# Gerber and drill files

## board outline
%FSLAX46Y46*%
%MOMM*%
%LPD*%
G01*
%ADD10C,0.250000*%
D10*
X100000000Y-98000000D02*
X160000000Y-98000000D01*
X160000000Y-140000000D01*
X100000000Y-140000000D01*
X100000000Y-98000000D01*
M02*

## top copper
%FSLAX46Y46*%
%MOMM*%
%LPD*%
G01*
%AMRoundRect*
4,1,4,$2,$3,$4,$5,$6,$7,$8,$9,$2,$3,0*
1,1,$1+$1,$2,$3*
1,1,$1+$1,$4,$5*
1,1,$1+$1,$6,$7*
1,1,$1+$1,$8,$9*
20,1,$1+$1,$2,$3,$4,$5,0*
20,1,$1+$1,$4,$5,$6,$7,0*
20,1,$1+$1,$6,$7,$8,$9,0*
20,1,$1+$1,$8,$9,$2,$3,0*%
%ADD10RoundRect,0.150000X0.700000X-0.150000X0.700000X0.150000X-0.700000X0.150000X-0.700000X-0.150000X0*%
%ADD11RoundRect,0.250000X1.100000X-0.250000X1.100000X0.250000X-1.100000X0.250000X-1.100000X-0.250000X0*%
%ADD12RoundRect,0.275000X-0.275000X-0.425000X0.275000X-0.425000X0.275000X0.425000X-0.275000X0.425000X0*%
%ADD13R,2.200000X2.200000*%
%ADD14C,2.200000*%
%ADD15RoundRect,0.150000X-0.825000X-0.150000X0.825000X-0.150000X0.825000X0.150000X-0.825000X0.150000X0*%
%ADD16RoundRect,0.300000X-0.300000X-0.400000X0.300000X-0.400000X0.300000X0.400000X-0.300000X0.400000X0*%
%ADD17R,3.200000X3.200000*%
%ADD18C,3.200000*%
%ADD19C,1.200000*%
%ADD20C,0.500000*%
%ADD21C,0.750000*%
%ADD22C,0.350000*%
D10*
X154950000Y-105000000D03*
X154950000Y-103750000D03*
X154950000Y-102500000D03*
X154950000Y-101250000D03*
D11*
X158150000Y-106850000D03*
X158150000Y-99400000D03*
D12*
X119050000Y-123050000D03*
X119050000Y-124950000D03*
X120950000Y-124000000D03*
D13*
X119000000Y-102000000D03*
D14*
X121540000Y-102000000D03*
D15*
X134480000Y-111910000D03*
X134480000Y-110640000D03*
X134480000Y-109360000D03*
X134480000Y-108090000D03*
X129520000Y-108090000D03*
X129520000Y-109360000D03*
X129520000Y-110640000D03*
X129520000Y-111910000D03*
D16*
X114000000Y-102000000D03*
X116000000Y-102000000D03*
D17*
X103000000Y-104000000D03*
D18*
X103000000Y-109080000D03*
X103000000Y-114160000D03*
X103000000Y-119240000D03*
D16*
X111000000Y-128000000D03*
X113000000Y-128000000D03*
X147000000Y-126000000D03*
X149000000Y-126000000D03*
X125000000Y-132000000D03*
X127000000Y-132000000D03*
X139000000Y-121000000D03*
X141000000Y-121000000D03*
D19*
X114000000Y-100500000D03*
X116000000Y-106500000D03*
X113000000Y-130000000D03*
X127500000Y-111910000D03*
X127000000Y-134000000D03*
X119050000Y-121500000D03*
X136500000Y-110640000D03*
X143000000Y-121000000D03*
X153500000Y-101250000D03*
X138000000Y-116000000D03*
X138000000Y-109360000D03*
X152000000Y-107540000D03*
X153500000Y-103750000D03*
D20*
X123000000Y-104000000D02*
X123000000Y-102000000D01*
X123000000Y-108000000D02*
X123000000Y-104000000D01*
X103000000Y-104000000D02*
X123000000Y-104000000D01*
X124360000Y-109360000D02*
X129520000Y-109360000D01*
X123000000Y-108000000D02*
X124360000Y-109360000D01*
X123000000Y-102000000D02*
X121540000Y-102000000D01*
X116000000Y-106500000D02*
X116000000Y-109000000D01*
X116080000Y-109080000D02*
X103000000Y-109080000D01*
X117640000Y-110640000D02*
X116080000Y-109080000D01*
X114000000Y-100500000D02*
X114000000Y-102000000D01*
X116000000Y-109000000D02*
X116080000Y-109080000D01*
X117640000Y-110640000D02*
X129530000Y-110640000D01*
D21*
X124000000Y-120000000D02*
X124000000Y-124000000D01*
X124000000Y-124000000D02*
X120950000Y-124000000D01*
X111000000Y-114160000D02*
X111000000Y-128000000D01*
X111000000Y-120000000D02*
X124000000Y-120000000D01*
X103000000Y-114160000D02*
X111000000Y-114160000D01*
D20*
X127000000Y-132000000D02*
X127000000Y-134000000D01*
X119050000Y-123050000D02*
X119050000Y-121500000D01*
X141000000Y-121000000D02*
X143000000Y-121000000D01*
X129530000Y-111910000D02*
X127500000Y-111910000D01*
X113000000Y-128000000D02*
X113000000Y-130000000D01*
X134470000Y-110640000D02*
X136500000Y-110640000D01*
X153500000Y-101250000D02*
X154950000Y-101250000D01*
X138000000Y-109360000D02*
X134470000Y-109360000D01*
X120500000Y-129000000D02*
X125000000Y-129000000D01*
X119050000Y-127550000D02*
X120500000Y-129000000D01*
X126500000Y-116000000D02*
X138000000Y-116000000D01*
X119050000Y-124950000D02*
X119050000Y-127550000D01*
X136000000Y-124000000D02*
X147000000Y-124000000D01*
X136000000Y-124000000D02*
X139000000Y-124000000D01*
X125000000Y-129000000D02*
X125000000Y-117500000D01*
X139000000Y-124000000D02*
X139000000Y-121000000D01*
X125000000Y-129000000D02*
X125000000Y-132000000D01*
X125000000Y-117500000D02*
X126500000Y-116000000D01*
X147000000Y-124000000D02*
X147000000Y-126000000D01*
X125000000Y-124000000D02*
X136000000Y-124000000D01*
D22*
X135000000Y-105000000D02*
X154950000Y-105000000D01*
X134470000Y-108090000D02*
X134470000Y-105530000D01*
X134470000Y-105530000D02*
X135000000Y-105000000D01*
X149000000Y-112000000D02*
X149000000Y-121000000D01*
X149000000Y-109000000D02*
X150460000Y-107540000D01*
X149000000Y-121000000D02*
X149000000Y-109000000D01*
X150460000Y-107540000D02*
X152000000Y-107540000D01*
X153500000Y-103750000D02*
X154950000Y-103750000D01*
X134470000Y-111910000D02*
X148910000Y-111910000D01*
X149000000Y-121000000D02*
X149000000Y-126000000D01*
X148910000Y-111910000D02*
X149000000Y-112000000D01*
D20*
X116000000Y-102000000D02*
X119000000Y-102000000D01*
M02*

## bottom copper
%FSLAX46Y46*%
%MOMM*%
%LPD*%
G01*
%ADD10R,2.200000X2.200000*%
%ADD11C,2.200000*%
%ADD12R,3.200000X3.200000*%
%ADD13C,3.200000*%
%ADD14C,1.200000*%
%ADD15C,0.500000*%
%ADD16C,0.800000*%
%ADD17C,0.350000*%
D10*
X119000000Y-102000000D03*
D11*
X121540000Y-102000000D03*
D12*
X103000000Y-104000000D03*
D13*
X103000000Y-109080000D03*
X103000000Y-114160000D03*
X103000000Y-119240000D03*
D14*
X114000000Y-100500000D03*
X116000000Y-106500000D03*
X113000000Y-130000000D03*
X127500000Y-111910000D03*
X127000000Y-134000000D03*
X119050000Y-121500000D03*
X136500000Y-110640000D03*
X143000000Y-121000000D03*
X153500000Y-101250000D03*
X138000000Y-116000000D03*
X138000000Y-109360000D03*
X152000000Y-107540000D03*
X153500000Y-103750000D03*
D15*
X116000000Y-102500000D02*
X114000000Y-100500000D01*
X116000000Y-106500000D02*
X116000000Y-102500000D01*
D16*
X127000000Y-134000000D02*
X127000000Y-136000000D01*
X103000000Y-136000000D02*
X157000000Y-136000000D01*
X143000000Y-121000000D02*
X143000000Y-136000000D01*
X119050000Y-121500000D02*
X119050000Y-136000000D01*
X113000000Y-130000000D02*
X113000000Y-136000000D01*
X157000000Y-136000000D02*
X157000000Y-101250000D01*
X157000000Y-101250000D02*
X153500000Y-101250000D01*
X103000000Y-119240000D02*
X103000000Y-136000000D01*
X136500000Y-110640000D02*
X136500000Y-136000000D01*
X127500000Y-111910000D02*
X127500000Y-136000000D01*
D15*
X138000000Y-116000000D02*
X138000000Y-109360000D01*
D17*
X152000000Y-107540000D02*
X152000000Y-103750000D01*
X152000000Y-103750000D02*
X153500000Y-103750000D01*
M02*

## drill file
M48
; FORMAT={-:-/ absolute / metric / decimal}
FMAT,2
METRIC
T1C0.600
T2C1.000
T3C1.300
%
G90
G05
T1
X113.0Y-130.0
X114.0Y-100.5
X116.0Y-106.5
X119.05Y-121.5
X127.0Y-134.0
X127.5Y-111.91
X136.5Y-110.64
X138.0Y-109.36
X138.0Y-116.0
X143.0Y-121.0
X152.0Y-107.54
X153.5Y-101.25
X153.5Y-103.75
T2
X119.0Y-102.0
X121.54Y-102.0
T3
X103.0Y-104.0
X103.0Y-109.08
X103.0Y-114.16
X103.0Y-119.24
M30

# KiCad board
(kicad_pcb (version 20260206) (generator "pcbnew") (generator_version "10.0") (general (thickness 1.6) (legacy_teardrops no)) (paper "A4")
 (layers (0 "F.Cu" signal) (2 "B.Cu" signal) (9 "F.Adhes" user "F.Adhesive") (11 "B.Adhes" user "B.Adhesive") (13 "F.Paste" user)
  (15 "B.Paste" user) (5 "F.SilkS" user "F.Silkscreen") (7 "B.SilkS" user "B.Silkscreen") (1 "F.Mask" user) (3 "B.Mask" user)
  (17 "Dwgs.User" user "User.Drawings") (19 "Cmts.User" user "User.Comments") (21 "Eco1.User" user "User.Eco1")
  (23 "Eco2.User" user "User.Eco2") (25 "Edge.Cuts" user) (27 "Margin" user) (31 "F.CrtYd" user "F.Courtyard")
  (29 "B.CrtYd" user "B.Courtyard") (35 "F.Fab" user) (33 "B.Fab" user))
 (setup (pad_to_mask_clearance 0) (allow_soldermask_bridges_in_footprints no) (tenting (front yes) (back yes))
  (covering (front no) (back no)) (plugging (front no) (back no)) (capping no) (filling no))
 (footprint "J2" (layer "F.Cu") (at 156.8 103.125 90)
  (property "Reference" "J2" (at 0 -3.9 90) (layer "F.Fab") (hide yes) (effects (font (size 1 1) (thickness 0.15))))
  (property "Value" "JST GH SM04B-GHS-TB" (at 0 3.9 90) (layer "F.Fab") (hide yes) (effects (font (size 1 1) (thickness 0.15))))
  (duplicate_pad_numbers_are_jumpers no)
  (pad "1" smd roundrect (at -1.875 -1.85 90) (size 0.6 1.7) (layers "F.Cu" "F.Mask" "F.Paste") (roundrect_rratio 0.25) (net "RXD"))
  (pad "2" smd roundrect (at -0.625 -1.85 90) (size 0.6 1.7) (layers "F.Cu" "F.Mask" "F.Paste") (roundrect_rratio 0.25) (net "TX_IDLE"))
  (pad "3" smd roundrect (at 0.625 -1.85 90) (size 0.6 1.7) (layers "F.Cu" "F.Mask" "F.Paste") (roundrect_rratio 0.25))
  (pad "4" smd roundrect (at 1.875 -1.85 90) (size 0.6 1.7) (layers "F.Cu" "F.Mask" "F.Paste") (roundrect_rratio 0.25) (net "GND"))
  (pad "MP" smd roundrect (at -3.725 1.35 90) (size 1 2.7) (layers "F.Cu" "F.Mask" "F.Paste") (roundrect_rratio 0.25))
  (pad "MP" smd roundrect (at 3.725 1.35 90) (size 1 2.7) (layers "F.Cu" "F.Mask" "F.Paste") (roundrect_rratio 0.25)))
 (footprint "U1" (layer "F.Cu") (at 120 124)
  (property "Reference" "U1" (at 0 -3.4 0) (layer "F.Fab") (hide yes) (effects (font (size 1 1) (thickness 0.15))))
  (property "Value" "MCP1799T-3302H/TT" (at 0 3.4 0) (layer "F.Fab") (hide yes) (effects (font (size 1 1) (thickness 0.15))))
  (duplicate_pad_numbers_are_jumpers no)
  (pad "1" smd roundrect (at -0.95 -0.95) (size 1.1 1.4) (layers "F.Cu" "F.Mask" "F.Paste") (roundrect_rratio 0.25) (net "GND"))
  (pad "2" smd roundrect (at -0.95 0.95) (size 1.1 1.4) (layers "F.Cu" "F.Mask" "F.Paste") (roundrect_rratio 0.25) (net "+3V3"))
  (pad "3" smd roundrect (at 0.95 0) (size 1.1 1.4) (layers "F.Cu" "F.Mask" "F.Paste") (roundrect_rratio 0.25) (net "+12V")))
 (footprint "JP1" (layer "F.Cu") (at 119 102)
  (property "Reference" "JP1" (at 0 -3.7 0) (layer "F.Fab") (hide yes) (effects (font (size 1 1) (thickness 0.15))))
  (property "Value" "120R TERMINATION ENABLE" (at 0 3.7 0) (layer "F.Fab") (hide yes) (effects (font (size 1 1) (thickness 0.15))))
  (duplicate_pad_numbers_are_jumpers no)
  (pad "1" thru_hole rect (at 0 0) (size 2.2 2.2) (drill 1) (layers "*.Cu" "*.Mask") (remove_unused_layers no) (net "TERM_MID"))
  (pad "2" thru_hole circle (at 2.54 0) (size 2.2 2.2) (drill 1) (layers "*.Cu" "*.Mask") (remove_unused_layers no) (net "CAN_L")))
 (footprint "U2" (layer "F.Cu") (at 132 110 180)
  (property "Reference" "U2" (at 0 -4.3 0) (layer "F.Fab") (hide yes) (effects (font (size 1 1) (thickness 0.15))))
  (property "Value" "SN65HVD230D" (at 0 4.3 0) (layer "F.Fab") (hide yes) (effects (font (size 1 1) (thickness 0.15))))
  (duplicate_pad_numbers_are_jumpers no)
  (pad "1" smd roundrect (at -2.48 -1.91) (size 1.95 0.6) (layers "F.Cu" "F.Mask" "F.Paste") (roundrect_rratio 0.25) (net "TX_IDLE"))
  (pad "2" smd roundrect (at -2.48 -0.64) (size 1.95 0.6) (layers "F.Cu" "F.Mask" "F.Paste") (roundrect_rratio 0.25) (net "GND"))
  (pad "3" smd roundrect (at -2.48 0.64) (size 1.95 0.6) (layers "F.Cu" "F.Mask" "F.Paste") (roundrect_rratio 0.25) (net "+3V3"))
  (pad "4" smd roundrect (at -2.48 1.91) (size 1.95 0.6) (layers "F.Cu" "F.Mask" "F.Paste") (roundrect_rratio 0.25) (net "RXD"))
  (pad "5" smd roundrect (at 2.48 1.91) (size 1.95 0.6) (layers "F.Cu" "F.Mask" "F.Paste") (roundrect_rratio 0.25))
  (pad "6" smd roundrect (at 2.48 0.64) (size 1.95 0.6) (layers "F.Cu" "F.Mask" "F.Paste") (roundrect_rratio 0.25) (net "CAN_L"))
  (pad "7" smd roundrect (at 2.48 -0.64) (size 1.95 0.6) (layers "F.Cu" "F.Mask" "F.Paste") (roundrect_rratio 0.25) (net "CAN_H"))
  (pad "8" smd roundrect (at 2.48 -1.91) (size 1.95 0.6) (layers "F.Cu" "F.Mask" "F.Paste") (roundrect_rratio 0.25) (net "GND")))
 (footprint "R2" (layer "F.Cu") (at 115 102)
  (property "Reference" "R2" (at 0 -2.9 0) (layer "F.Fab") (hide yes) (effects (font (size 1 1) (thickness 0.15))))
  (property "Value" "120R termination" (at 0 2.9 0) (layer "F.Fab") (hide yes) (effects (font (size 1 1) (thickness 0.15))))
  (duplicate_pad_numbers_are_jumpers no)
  (pad "1" smd roundrect (at -1 0) (size 1.2 1.4) (layers "F.Cu" "F.Mask" "F.Paste") (roundrect_rratio 0.25) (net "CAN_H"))
  (pad "2" smd roundrect (at 1 0) (size 1.2 1.4) (layers "F.Cu" "F.Mask" "F.Paste") (roundrect_rratio 0.25) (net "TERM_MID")))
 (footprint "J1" (layer "F.Cu") (at 103 104)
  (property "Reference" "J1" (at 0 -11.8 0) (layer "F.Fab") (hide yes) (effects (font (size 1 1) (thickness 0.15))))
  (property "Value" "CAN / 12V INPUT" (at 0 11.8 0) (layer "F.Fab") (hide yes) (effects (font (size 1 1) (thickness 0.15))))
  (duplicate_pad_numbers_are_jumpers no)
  (pad "1" thru_hole rect (at 0 0) (size 3.2 3.2) (drill 1.3) (layers "*.Cu" "*.Mask") (remove_unused_layers no) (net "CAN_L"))
  (pad "2" thru_hole circle (at 0 5.08) (size 3.2 3.2) (drill 1.3) (layers "*.Cu" "*.Mask") (remove_unused_layers no) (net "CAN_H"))
  (pad "3" thru_hole circle (at 0 10.16) (size 3.2 3.2) (drill 1.3) (layers "*.Cu" "*.Mask") (remove_unused_layers no) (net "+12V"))
  (pad "4" thru_hole circle (at 0 15.24) (size 3.2 3.2) (drill 1.3) (layers "*.Cu" "*.Mask") (remove_unused_layers no) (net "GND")))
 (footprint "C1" (layer "F.Cu") (at 112 128)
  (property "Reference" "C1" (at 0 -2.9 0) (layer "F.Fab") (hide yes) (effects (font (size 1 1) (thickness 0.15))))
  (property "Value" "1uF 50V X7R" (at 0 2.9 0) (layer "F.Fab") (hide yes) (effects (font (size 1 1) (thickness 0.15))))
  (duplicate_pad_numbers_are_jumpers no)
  (pad "1" smd roundrect (at -1 0) (size 1.2 1.4) (layers "F.Cu" "F.Mask" "F.Paste") (roundrect_rratio 0.25) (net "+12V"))
  (pad "2" smd roundrect (at 1 0) (size 1.2 1.4) (layers "F.Cu" "F.Mask" "F.Paste") (roundrect_rratio 0.25) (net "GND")))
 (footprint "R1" (layer "F.Cu") (at 148 126)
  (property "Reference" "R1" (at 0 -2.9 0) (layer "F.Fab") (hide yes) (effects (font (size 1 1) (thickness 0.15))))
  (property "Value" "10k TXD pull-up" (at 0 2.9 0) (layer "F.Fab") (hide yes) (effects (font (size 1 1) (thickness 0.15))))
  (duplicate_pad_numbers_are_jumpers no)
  (pad "1" smd roundrect (at -1 0) (size 1.2 1.4) (layers "F.Cu" "F.Mask" "F.Paste") (roundrect_rratio 0.25) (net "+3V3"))
  (pad "2" smd roundrect (at 1 0) (size 1.2 1.4) (layers "F.Cu" "F.Mask" "F.Paste") (roundrect_rratio 0.25) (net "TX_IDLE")))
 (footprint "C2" (layer "F.Cu") (at 126 132)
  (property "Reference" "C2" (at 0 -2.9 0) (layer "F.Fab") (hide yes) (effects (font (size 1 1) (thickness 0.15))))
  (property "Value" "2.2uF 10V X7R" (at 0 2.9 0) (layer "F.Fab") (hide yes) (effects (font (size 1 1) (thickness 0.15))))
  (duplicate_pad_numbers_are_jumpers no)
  (pad "1" smd roundrect (at -1 0) (size 1.2 1.4) (layers "F.Cu" "F.Mask" "F.Paste") (roundrect_rratio 0.25) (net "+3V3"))
  (pad "2" smd roundrect (at 1 0) (size 1.2 1.4) (layers "F.Cu" "F.Mask" "F.Paste") (roundrect_rratio 0.25) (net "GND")))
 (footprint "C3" (layer "F.Cu") (at 140 121)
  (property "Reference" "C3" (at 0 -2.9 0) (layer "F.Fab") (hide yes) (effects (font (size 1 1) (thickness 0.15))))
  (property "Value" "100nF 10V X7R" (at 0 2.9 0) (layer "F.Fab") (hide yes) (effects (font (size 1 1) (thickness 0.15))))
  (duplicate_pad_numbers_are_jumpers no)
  (pad "1" smd roundrect (at -1 0) (size 1.2 1.4) (layers "F.Cu" "F.Mask" "F.Paste") (roundrect_rratio 0.25) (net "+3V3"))
  (pad "2" smd roundrect (at 1 0) (size 1.2 1.4) (layers "F.Cu" "F.Mask" "F.Paste") (roundrect_rratio 0.25) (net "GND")))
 (gr_rect (start 100 98) (end 160 140) (stroke (width 0.25) (type default)) (fill no) (layer "Edge.Cuts"))
 (segment (start 123 104) (end 123 102) (width 0.5) (layer "F.Cu") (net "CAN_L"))
 (segment (start 123 108) (end 123 104) (width 0.5) (layer "F.Cu") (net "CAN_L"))
 (segment (start 103 104) (end 123 104) (width 0.5) (layer "F.Cu") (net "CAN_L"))
 (segment (start 124.36 109.36) (end 129.52 109.36) (width 0.5) (layer "F.Cu") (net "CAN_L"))
 (segment (start 123 108) (end 124.36 109.36) (width 0.5) (layer "F.Cu") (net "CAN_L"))
 (segment (start 123 102) (end 121.54 102) (width 0.5) (layer "F.Cu") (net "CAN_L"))
 (segment (start 116 106.5) (end 116 109) (width 0.5) (layer "F.Cu") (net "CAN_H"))
 (segment (start 116.08 109.08) (end 103 109.08) (width 0.5) (layer "F.Cu") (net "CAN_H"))
 (segment (start 117.64 110.64) (end 116.08 109.08) (width 0.5) (layer "F.Cu") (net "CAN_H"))
 (segment (start 114 100.5) (end 114 102) (width 0.5) (layer "F.Cu") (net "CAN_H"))
 (segment (start 116 109) (end 116.08 109.08) (width 0.5) (layer "F.Cu") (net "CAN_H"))
 (segment (start 117.64 110.64) (end 129.53 110.64) (width 0.5) (layer "F.Cu") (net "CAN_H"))
 (via (at 114 100.5) (size 1.2) (drill 0.6) (layers "F.Cu" "B.Cu") (capping no) (covering (front no) (back no))
  (plugging (front no) (back no)) (filling no) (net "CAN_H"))
 (via (at 116 106.5) (size 1.2) (drill 0.6) (layers "F.Cu" "B.Cu") (capping no) (covering (front no) (back no))
  (plugging (front no) (back no)) (filling no) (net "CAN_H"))
 (segment (start 116 102.5) (end 114 100.5) (width 0.5) (layer "B.Cu") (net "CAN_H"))
 (segment (start 116 106.5) (end 116 102.5) (width 0.5) (layer "B.Cu") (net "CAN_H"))
 (segment (start 124 120) (end 124 124) (width 0.75) (layer "F.Cu") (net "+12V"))
 (segment (start 124 124) (end 120.95 124) (width 0.75) (layer "F.Cu") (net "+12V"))
 (segment (start 111 114.16) (end 111 128) (width 0.75) (layer "F.Cu") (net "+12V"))
 (segment (start 111 120) (end 124 120) (width 0.75) (layer "F.Cu") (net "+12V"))
 (segment (start 103 114.16) (end 111 114.16) (width 0.75) (layer "F.Cu") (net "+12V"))
 (segment (start 127 132) (end 127 134) (width 0.5) (layer "F.Cu") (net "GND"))
 (segment (start 119.05 123.05) (end 119.05 121.5) (width 0.5) (layer "F.Cu") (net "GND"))
 (segment (start 141 121) (end 143 121) (width 0.5) (layer "F.Cu") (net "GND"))
 (segment (start 129.53 111.91) (end 127.5 111.91) (width 0.5) (layer "F.Cu") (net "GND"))
 (segment (start 113 128) (end 113 130) (width 0.5) (layer "F.Cu") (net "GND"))
 (segment (start 134.47 110.64) (end 136.5 110.64) (width 0.5) (layer "F.Cu") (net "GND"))
 (via (at 113 130) (size 1.2) (drill 0.6) (layers "F.Cu" "B.Cu") (capping no) (covering (front no) (back no))
  (plugging (front no) (back no)) (filling no) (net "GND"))
 (via (at 127.5 111.91) (size 1.2) (drill 0.6) (layers "F.Cu" "B.Cu") (capping no) (covering (front no) (back no))
  (plugging (front no) (back no)) (filling no) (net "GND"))
 (via (at 127 134) (size 1.2) (drill 0.6) (layers "F.Cu" "B.Cu") (capping no) (covering (front no) (back no))
  (plugging (front no) (back no)) (filling no) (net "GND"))
 (via (at 119.05 121.5) (size 1.2) (drill 0.6) (layers "F.Cu" "B.Cu") (capping no) (covering (front no) (back no))
  (plugging (front no) (back no)) (filling no) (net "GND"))
 (via (at 136.5 110.64) (size 1.2) (drill 0.6) (layers "F.Cu" "B.Cu") (capping no) (covering (front no) (back no))
  (plugging (front no) (back no)) (filling no) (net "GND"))
 (via (at 143 121) (size 1.2) (drill 0.6) (layers "F.Cu" "B.Cu") (capping no) (covering (front no) (back no))
  (plugging (front no) (back no)) (filling no) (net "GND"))
 (segment (start 127 134) (end 127 136) (width 0.8) (layer "B.Cu") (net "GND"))
 (segment (start 103 136) (end 157 136) (width 0.8) (layer "B.Cu") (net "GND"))
 (segment (start 143 121) (end 143 136) (width 0.8) (layer "B.Cu") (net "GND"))
 (segment (start 119.05 121.5) (end 119.05 136) (width 0.8) (layer "B.Cu") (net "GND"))
 (segment (start 113 130) (end 113 136) (width 0.8) (layer "B.Cu") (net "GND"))
 (segment (start 157 136) (end 157 101.25) (width 0.8) (layer "B.Cu") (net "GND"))
 (segment (start 157 101.25) (end 153.5 101.25) (width 0.8) (layer "B.Cu") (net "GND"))
 (via (at 153.5 101.25) (size 1.2) (drill 0.6) (layers "F.Cu" "B.Cu") (capping no) (covering (front no) (back no))
  (plugging (front no) (back no)) (filling no) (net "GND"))
 (segment (start 153.5 101.25) (end 154.95 101.25) (width 0.5) (layer "F.Cu") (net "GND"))
 (segment (start 103 119.24) (end 103 136) (width 0.8) (layer "B.Cu") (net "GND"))
 (segment (start 136.5 110.64) (end 136.5 136) (width 0.8) (layer "B.Cu") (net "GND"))
 (segment (start 127.5 111.91) (end 127.5 136) (width 0.8) (layer "B.Cu") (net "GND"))
 (segment (start 138 109.36) (end 134.47 109.36) (width 0.5) (layer "F.Cu") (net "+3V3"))
 (segment (start 120.5 129) (end 125 129) (width 0.5) (layer "F.Cu") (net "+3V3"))
 (segment (start 119.05 127.55) (end 120.5 129) (width 0.5) (layer "F.Cu") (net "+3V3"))
 (segment (start 126.5 116) (end 138 116) (width 0.5) (layer "F.Cu") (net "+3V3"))
 (segment (start 119.05 124.95) (end 119.05 127.55) (width 0.5) (layer "F.Cu") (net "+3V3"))
 (segment (start 136 124) (end 147 124) (width 0.5) (layer "F.Cu") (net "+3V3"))
 (segment (start 136 124) (end 139 124) (width 0.5) (layer "F.Cu") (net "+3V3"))
 (segment (start 125 129) (end 125 117.5) (width 0.5) (layer "F.Cu") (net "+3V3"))
 (segment (start 139 124) (end 139 121) (width 0.5) (layer "F.Cu") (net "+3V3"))
 (segment (start 125 129) (end 125 132) (width 0.5) (layer "F.Cu") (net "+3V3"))
 (segment (start 125 117.5) (end 126.5 116) (width 0.5) (layer "F.Cu") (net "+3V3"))
 (segment (start 147 124) (end 147 126) (width 0.5) (layer "F.Cu") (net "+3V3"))
 (segment (start 125 124) (end 136 124) (width 0.5) (layer "F.Cu") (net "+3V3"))
 (via (at 138 116) (size 1.2) (drill 0.6) (layers "F.Cu" "B.Cu") (capping no) (covering (front no) (back no))
  (plugging (front no) (back no)) (filling no) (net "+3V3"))
 (via (at 138 109.36) (size 1.2) (drill 0.6) (layers "F.Cu" "B.Cu") (capping no) (covering (front no) (back no))
  (plugging (front no) (back no)) (filling no) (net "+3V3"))
 (segment (start 138 116) (end 138 109.36) (width 0.5) (layer "B.Cu") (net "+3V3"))
 (segment (start 135 105) (end 154.95 105) (width 0.35) (layer "F.Cu") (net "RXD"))
 (segment (start 134.47 108.09) (end 134.47 105.53) (width 0.35) (layer "F.Cu") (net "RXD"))
 (segment (start 134.47 105.53) (end 135 105) (width 0.35) (layer "F.Cu") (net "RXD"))
 (segment (start 149 112) (end 149 121) (width 0.35) (layer "F.Cu") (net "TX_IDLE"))
 (segment (start 149 109) (end 150.46 107.54) (width 0.35) (layer "F.Cu") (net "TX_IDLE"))
 (segment (start 149 121) (end 149 109) (width 0.35) (layer "F.Cu") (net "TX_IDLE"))
 (segment (start 150.46 107.54) (end 152 107.54) (width 0.35) (layer "F.Cu") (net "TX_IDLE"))
 (via (at 152 107.54) (size 1.2) (drill 0.6) (layers "F.Cu" "B.Cu") (capping no) (covering (front no) (back no))
  (plugging (front no) (back no)) (filling no) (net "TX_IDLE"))
 (segment (start 152 107.54) (end 152 103.75) (width 0.35) (layer "B.Cu") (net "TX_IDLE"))
 (segment (start 152 103.75) (end 153.5 103.75) (width 0.35) (layer "B.Cu") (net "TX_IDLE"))
 (via (at 153.5 103.75) (size 1.2) (drill 0.6) (layers "F.Cu" "B.Cu") (capping no) (covering (front no) (back no))
  (plugging (front no) (back no)) (filling no) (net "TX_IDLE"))
 (segment (start 153.5 103.75) (end 154.95 103.75) (width 0.35) (layer "F.Cu") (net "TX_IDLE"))
 (segment (start 134.47 111.91) (end 148.91 111.91) (width 0.35) (layer "F.Cu") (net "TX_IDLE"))
 (segment (start 149 121) (end 149 126) (width 0.35) (layer "F.Cu") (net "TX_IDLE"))
 (segment (start 148.91 111.91) (end 149 112) (width 0.35) (layer "F.Cu") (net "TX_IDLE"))
 (segment (start 116 102) (end 119 102) (width 0.5) (layer "F.Cu") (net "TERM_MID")))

